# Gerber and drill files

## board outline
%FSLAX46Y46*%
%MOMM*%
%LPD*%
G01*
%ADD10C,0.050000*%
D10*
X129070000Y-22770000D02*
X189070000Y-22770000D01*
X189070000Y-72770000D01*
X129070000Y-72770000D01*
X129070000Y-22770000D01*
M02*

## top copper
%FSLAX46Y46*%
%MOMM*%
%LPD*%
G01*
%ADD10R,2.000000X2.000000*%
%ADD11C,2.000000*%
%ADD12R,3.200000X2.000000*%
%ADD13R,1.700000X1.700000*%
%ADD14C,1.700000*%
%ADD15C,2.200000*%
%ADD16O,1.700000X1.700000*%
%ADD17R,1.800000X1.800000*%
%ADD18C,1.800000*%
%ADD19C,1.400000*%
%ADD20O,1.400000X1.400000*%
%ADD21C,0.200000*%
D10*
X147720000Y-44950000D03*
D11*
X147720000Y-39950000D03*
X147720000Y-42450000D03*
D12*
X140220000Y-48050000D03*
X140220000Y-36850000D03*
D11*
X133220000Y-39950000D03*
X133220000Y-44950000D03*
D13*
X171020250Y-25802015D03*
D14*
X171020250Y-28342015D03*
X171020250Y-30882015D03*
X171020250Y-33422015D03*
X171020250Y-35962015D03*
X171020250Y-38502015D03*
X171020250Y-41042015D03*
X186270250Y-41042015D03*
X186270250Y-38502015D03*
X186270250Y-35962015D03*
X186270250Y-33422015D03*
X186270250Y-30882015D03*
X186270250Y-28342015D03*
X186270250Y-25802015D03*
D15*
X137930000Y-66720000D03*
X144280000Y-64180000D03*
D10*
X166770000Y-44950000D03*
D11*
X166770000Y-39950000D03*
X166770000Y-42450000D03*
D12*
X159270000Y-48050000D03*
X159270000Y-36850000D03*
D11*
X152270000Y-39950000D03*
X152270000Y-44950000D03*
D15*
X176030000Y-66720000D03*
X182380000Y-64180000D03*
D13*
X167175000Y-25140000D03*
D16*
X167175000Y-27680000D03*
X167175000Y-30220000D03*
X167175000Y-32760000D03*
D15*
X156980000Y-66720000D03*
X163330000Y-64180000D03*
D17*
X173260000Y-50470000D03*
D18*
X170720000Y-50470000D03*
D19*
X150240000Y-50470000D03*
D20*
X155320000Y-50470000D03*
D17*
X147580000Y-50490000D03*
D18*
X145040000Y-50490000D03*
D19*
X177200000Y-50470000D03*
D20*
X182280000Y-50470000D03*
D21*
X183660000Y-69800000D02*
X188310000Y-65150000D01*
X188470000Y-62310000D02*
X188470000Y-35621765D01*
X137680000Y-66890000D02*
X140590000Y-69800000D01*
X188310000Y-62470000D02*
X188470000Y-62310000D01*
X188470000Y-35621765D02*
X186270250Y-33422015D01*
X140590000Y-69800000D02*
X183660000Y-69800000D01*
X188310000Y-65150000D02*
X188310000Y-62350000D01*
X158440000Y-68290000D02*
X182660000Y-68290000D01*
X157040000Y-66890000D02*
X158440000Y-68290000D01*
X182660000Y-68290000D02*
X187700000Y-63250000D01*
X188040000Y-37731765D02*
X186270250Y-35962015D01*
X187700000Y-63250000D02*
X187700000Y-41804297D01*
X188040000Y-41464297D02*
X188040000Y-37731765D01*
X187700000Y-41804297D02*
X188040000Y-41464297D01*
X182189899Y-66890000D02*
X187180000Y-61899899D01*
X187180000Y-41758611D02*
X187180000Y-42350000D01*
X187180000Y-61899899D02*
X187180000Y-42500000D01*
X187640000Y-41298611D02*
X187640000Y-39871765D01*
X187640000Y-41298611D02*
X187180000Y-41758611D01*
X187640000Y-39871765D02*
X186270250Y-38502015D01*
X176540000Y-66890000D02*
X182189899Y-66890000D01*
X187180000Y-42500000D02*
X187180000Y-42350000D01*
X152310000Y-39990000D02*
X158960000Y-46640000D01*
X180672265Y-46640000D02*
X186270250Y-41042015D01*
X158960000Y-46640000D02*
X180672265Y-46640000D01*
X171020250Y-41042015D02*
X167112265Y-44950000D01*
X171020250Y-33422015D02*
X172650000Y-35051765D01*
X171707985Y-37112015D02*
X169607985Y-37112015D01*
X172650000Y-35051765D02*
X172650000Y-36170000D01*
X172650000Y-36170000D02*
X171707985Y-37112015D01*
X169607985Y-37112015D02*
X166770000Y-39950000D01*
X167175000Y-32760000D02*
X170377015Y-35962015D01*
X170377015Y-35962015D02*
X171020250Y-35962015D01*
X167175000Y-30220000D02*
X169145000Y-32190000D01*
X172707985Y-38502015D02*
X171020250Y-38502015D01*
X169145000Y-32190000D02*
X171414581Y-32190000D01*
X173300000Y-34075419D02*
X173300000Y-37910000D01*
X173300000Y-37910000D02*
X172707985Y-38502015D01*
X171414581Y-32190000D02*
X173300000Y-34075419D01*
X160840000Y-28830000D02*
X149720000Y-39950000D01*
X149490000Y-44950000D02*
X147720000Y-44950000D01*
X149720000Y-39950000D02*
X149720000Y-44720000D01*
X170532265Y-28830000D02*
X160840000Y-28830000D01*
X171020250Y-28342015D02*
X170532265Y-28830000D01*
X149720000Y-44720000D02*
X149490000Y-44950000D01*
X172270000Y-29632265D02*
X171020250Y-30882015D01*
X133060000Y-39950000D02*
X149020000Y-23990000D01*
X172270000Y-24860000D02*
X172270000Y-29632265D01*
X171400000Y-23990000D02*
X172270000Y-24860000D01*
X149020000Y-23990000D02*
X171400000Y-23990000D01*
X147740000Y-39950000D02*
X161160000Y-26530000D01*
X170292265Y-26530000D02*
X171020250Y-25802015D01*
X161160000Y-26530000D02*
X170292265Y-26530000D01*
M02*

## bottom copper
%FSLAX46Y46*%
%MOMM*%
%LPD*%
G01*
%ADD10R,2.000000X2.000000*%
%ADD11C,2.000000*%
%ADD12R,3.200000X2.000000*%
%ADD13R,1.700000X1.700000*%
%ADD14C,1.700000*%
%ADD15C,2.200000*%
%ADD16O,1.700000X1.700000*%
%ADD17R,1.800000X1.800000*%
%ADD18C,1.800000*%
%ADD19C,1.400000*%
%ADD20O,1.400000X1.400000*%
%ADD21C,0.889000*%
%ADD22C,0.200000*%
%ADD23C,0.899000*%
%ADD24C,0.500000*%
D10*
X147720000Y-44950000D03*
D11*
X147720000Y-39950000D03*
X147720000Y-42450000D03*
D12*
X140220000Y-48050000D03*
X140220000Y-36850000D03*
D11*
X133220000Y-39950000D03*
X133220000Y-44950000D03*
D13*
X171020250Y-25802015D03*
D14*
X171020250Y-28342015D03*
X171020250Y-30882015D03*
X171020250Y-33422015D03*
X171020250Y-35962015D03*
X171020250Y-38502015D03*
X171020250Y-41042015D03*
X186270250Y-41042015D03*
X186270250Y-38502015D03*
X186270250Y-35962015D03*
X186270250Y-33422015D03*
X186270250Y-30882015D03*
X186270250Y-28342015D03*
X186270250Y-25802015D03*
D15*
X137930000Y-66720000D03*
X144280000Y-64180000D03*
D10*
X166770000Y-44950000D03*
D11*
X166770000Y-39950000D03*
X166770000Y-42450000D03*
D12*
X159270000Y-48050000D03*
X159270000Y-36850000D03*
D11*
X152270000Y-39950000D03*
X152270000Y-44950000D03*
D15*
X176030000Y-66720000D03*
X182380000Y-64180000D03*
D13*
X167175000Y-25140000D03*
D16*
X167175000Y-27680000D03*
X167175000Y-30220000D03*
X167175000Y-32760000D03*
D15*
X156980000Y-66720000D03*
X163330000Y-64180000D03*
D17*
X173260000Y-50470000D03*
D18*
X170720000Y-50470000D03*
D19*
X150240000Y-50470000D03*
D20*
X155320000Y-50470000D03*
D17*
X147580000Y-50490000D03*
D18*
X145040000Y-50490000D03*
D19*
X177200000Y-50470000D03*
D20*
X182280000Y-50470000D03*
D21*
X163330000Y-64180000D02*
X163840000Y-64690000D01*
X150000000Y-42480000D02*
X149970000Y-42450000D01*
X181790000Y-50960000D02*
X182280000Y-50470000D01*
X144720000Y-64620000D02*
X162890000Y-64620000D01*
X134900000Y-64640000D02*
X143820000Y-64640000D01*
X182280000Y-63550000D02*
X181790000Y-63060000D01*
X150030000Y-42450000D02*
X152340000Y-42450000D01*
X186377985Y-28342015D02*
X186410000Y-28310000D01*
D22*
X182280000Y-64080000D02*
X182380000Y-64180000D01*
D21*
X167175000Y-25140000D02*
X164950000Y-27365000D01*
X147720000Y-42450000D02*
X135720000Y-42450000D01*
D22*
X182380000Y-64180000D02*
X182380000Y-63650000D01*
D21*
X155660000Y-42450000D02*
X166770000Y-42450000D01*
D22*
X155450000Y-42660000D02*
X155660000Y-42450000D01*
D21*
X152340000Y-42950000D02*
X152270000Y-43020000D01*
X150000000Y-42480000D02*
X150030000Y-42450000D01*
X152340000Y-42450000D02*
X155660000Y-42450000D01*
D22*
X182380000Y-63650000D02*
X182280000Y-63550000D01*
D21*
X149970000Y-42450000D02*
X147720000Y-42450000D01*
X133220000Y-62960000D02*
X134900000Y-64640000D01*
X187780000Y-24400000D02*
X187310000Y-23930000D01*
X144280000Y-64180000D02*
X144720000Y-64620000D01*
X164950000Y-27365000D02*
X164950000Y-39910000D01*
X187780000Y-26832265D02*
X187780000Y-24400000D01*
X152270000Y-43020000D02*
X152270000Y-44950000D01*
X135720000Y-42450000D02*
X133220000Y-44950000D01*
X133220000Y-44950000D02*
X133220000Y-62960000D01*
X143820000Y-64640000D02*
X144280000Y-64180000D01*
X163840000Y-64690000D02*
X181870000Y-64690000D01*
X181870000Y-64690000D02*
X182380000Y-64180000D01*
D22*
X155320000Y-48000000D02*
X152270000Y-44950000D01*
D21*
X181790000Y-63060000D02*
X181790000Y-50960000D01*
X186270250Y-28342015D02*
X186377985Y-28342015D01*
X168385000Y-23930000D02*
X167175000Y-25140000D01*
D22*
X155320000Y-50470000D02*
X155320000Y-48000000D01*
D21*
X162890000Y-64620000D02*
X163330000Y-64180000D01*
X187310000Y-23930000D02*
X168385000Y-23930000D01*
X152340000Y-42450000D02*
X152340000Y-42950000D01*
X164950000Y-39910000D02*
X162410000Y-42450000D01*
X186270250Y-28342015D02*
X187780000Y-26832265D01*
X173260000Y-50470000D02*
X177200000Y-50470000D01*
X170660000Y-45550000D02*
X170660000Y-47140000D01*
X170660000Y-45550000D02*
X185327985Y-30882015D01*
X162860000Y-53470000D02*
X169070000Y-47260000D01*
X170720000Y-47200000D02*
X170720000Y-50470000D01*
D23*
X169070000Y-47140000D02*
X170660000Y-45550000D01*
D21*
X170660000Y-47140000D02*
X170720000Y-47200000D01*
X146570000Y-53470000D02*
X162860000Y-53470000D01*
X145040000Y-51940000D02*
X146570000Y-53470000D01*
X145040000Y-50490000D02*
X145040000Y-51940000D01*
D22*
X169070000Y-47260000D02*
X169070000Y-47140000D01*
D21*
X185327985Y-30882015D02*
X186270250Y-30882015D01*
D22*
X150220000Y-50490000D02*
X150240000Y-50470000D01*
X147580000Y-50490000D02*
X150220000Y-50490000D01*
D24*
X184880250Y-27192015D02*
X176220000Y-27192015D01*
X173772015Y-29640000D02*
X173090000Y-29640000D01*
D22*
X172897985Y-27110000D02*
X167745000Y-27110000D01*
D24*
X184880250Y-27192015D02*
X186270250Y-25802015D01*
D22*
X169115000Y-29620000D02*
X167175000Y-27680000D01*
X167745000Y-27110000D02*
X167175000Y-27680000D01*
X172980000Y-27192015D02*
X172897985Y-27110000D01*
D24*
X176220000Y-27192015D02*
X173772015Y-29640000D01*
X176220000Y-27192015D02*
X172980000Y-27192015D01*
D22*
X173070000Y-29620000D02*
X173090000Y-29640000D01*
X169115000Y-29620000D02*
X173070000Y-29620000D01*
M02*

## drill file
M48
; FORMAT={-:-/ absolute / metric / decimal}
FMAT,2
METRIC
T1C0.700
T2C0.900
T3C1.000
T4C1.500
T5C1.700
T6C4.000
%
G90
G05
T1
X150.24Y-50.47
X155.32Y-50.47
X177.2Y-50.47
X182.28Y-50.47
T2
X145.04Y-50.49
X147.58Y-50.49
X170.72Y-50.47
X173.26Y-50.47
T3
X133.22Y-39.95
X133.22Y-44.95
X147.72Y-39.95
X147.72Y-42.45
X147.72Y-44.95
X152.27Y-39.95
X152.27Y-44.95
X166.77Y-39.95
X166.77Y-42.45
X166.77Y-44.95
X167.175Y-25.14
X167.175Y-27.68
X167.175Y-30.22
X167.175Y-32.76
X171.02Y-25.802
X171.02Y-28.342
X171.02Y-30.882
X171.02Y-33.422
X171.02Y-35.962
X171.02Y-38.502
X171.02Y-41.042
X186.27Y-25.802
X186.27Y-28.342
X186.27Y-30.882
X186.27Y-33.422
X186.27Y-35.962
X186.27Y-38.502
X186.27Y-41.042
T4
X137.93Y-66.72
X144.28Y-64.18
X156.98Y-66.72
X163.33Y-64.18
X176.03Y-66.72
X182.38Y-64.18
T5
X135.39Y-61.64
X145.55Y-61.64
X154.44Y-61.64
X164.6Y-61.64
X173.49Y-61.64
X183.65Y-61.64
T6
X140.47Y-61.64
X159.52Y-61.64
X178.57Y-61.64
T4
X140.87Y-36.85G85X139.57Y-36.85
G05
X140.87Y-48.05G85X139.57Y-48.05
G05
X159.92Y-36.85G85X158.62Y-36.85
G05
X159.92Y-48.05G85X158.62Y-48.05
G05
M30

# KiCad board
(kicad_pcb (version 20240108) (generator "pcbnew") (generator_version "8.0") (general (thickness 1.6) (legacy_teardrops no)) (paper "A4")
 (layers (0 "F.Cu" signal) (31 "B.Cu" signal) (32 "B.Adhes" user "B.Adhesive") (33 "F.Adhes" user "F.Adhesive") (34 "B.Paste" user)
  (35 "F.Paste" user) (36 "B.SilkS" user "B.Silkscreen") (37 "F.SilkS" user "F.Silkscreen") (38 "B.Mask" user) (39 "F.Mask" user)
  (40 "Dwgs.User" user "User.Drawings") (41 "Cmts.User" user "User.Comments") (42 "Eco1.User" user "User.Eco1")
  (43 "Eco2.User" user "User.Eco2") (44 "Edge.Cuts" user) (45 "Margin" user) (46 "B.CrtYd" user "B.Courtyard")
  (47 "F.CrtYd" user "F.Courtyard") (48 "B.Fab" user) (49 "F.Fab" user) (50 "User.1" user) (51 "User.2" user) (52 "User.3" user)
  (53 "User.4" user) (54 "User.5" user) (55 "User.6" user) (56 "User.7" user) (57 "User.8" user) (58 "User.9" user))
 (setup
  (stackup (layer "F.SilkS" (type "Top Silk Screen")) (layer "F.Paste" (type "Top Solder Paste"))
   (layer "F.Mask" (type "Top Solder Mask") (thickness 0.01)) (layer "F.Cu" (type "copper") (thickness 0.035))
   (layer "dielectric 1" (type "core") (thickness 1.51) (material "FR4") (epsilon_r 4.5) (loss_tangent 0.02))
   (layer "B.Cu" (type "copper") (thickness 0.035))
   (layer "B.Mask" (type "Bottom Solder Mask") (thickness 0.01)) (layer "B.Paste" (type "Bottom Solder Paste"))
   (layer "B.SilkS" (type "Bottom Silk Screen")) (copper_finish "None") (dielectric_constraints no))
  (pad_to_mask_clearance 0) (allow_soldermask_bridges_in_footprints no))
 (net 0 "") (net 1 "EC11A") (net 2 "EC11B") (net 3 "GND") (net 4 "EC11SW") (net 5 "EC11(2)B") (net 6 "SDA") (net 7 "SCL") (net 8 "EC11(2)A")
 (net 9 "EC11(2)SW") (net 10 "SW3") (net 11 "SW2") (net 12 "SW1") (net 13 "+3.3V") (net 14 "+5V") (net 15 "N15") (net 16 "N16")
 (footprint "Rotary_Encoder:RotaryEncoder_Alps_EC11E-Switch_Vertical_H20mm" (layer "F.Cu") (at 147.72 44.95 180)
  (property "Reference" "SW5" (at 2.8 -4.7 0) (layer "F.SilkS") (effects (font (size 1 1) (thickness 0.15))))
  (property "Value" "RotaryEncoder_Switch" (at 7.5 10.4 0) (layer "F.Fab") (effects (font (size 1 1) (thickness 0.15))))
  (pad "A" thru_hole rect (at 0 0 180) (size 2 2) (drill 1) (layers "*.Cu" "*.Mask") (remove_unused_layers no) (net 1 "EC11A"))
  (pad "B" thru_hole circle (at 0 5 180) (size 2 2) (drill 1) (layers "*.Cu" "*.Mask") (remove_unused_layers no) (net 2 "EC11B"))
  (pad "C" thru_hole circle (at 0 2.5 180) (size 2 2) (drill 1) (layers "*.Cu" "*.Mask") (remove_unused_layers no) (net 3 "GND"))
  (pad "MP" thru_hole rect (at 7.5 -3.1 180) (size 3.2 2) (drill oval 2.8 1.5) (layers "*.Cu" "*.Mask") (remove_unused_layers no))
  (pad "MP" thru_hole rect (at 7.5 8.1 180) (size 3.2 2) (drill oval 2.8 1.5) (layers "*.Cu" "*.Mask") (remove_unused_layers no))
  (pad "S1" thru_hole circle (at 14.5 5 180) (size 2 2) (drill 1) (layers "*.Cu" "*.Mask") (remove_unused_layers no) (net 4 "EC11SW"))
  (pad "S2" thru_hole circle (at 14.5 0 180) (size 2 2) (drill 1) (layers "*.Cu" "*.Mask") (remove_unused_layers no) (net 3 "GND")))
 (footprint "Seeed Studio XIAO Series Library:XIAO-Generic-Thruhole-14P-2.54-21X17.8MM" (layer "F.Cu") (at 178.64525 33.422015)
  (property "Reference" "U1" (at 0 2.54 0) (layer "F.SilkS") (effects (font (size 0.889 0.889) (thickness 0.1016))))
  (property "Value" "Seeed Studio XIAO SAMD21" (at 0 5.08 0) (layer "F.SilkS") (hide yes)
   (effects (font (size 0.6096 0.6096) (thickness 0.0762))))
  (pad "1" thru_hole rect (at -7.625 -7.62) (size 1.7 1.7) (drill 1) (layers "*.Cu" "*.Mask") (remove_unused_layers no) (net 2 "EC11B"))
  (pad "2" thru_hole circle (at -7.625 -5.08) (size 1.7 1.7) (drill 1) (layers "*.Cu" "*.Mask") (remove_unused_layers no) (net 1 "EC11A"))
  (pad "3" thru_hole circle (at -7.625 -2.54) (size 1.7 1.7) (drill 1) (layers "*.Cu" "*.Mask") (remove_unused_layers no) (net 4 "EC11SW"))
  (pad "4" thru_hole circle (at -7.625 0) (size 1.7 1.7) (drill 1) (layers "*.Cu" "*.Mask") (remove_unused_layers no) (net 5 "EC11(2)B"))
  (pad "5" thru_hole circle (at -7.625 2.54) (size 1.7 1.7) (drill 1) (layers "*.Cu" "*.Mask") (remove_unused_layers no) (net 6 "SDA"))
  (pad "6" thru_hole circle (at -7.625 5.08 180) (size 1.7 1.7) (drill 1) (layers "*.Cu" "*.Mask") (remove_unused_layers no) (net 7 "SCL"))
  (pad "7" thru_hole circle (at -7.625 7.62) (size 1.7 1.7) (drill 1) (layers "*.Cu" "*.Mask") (remove_unused_layers no) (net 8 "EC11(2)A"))
  (pad "8" thru_hole circle (at 7.625 7.62) (size 1.7 1.7) (drill 1) (layers "*.Cu" "*.Mask") (remove_unused_layers no) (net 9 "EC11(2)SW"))
  (pad "9" thru_hole circle (at 7.625 5.08) (size 1.7 1.7) (drill 1) (layers "*.Cu" "*.Mask") (remove_unused_layers no) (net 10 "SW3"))
  (pad "10" thru_hole circle (at 7.625 2.54) (size 1.7 1.7) (drill 1) (layers "*.Cu" "*.Mask") (remove_unused_layers no) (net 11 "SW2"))
  (pad "11" thru_hole circle (at 7.625 0) (size 1.7 1.7) (drill 1) (layers "*.Cu" "*.Mask") (remove_unused_layers no) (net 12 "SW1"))
  (pad "12" thru_hole circle (at 7.625 -2.54) (size 1.7 1.7) (drill 1) (layers "*.Cu" "*.Mask") (remove_unused_layers no) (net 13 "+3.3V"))
  (pad "13" thru_hole circle (at 7.625 -5.08) (size 1.7 1.7) (drill 1) (layers "*.Cu" "*.Mask") (remove_unused_layers no) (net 3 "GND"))
  (pad "14" thru_hole circle (at 7.625 -7.62) (size 1.7 1.7) (drill 1) (layers "*.Cu" "*.Mask") (remove_unused_layers no) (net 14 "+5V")))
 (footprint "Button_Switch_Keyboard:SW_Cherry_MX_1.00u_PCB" (layer "F.Cu") (at 137.93 66.72 180)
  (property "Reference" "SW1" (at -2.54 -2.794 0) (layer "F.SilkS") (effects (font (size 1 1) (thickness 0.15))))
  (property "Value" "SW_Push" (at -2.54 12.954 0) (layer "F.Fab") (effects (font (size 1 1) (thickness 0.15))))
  (pad "" np_thru_hole circle (at -7.62 5.08 180) (size 1.7 1.7) (drill 1.7) (layers "*.Cu" "*.Mask"))
  (pad "" np_thru_hole circle (at -2.54 5.08 180) (size 4 4) (drill 4) (layers "*.Cu" "*.Mask"))
  (pad "" np_thru_hole circle (at 2.54 5.08 180) (size 1.7 1.7) (drill 1.7) (layers "*.Cu" "*.Mask"))
  (pad "1" thru_hole circle (at 0 0 180) (size 2.2 2.2) (drill 1.5) (layers "*.Cu" "*.Mask") (remove_unused_layers no) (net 12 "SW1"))
  (pad "2" thru_hole circle (at -6.35 2.54 180) (size 2.2 2.2) (drill 1.5) (layers "*.Cu" "*.Mask") (remove_unused_layers no) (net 3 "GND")))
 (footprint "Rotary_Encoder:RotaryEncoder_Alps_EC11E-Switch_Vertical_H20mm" (layer "F.Cu") (at 166.77 44.95 180)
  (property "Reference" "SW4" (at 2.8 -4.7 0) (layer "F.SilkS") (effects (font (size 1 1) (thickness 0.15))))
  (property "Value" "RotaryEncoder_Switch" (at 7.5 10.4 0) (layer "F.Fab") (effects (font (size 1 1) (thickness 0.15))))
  (pad "A" thru_hole rect (at 0 0 180) (size 2 2) (drill 1) (layers "*.Cu" "*.Mask") (remove_unused_layers no) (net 8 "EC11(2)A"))
  (pad "B" thru_hole circle (at 0 5 180) (size 2 2) (drill 1) (layers "*.Cu" "*.Mask") (remove_unused_layers no) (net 5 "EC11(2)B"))
  (pad "C" thru_hole circle (at 0 2.5 180) (size 2 2) (drill 1) (layers "*.Cu" "*.Mask") (remove_unused_layers no) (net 3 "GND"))
  (pad "MP" thru_hole rect (at 7.5 -3.1 180) (size 3.2 2) (drill oval 2.8 1.5) (layers "*.Cu" "*.Mask") (remove_unused_layers no))
  (pad "MP" thru_hole rect (at 7.5 8.1 180) (size 3.2 2) (drill oval 2.8 1.5) (layers "*.Cu" "*.Mask") (remove_unused_layers no))
  (pad "S1" thru_hole circle (at 14.5 5 180) (size 2 2) (drill 1) (layers "*.Cu" "*.Mask") (remove_unused_layers no) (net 9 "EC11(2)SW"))
  (pad "S2" thru_hole circle (at 14.5 0 180) (size 2 2) (drill 1) (layers "*.Cu" "*.Mask") (remove_unused_layers no) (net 3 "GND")))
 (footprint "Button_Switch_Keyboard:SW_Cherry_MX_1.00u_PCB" (layer "F.Cu") (at 176.03 66.72 180)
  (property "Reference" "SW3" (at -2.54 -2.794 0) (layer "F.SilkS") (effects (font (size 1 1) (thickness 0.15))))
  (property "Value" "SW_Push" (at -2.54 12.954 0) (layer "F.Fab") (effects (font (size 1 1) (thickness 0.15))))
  (pad "" np_thru_hole circle (at -7.62 5.08 180) (size 1.7 1.7) (drill 1.7) (layers "*.Cu" "*.Mask"))
  (pad "" np_thru_hole circle (at -2.54 5.08 180) (size 4 4) (drill 4) (layers "*.Cu" "*.Mask"))
  (pad "" np_thru_hole circle (at 2.54 5.08 180) (size 1.7 1.7) (drill 1.7) (layers "*.Cu" "*.Mask"))
  (pad "1" thru_hole circle (at 0 0 180) (size 2.2 2.2) (drill 1.5) (layers "*.Cu" "*.Mask") (remove_unused_layers no) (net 10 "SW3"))
  (pad "2" thru_hole circle (at -6.35 2.54 180) (size 2.2 2.2) (drill 1.5) (layers "*.Cu" "*.Mask") (remove_unused_layers no) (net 3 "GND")))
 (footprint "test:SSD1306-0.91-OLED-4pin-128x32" (layer "F.Cu") (at 130.675 22.95)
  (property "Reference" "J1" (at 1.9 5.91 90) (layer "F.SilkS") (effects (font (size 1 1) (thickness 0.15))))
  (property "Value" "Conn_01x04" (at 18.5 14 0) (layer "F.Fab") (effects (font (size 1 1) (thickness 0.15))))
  (pad "1" thru_hole rect (at 36.5 2.19) (size 1.7 1.7) (drill 1) (layers "*.Cu" "*.Mask") (remove_unused_layers no) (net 3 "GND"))
  (pad "2" thru_hole oval (at 36.5 4.73) (size 1.7 1.7) (drill 1) (layers "*.Cu" "*.Mask") (remove_unused_layers no) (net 14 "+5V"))
  (pad "3" thru_hole oval (at 36.5 7.27) (size 1.7 1.7) (drill 1) (layers "*.Cu" "*.Mask") (remove_unused_layers no) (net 7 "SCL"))
  (pad "4" thru_hole oval (at 36.5 9.81) (size 1.7 1.7) (drill 1) (layers "*.Cu" "*.Mask") (remove_unused_layers no) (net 6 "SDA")))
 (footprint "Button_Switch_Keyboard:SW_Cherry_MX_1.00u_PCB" (layer "F.Cu") (at 156.98 66.72 180)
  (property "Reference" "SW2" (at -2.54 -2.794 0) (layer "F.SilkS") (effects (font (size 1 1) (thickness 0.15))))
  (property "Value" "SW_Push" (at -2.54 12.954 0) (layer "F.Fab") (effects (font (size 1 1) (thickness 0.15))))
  (pad "" np_thru_hole circle (at -7.62 5.08 180) (size 1.7 1.7) (drill 1.7) (layers "*.Cu" "*.Mask"))
  (pad "" np_thru_hole circle (at -2.54 5.08 180) (size 4 4) (drill 4) (layers "*.Cu" "*.Mask"))
  (pad "" np_thru_hole circle (at 2.54 5.08 180) (size 1.7 1.7) (drill 1.7) (layers "*.Cu" "*.Mask"))
  (pad "1" thru_hole circle (at 0 0 180) (size 2.2 2.2) (drill 1.5) (layers "*.Cu" "*.Mask") (remove_unused_layers no) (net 11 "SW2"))
  (pad "2" thru_hole circle (at -6.35 2.54 180) (size 2.2 2.2) (drill 1.5) (layers "*.Cu" "*.Mask") (remove_unused_layers no) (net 3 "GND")))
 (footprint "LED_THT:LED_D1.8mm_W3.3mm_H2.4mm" (layer "B.Cu") (at 173.26 50.47 180)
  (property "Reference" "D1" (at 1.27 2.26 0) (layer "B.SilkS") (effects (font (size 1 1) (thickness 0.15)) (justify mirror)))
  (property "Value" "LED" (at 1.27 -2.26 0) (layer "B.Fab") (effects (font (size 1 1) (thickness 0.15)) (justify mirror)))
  (pad "1" thru_hole rect (at 0 0 180) (size 1.8 1.8) (drill 0.9) (layers "*.Cu" "*.Mask") (remove_unused_layers no) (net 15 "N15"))
  (pad "2" thru_hole circle (at 2.54 0 180) (size 1.8 1.8) (drill 0.9) (layers "*.Cu" "*.Mask") (remove_unused_layers no) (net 13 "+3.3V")))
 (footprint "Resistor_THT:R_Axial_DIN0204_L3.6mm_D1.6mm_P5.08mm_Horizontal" (layer "B.Cu") (at 150.24 50.47)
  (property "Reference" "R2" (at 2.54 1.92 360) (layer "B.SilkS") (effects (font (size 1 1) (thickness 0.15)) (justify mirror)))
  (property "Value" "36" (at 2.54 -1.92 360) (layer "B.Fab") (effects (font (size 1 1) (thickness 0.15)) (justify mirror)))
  (pad "1" thru_hole circle (at 0 0) (size 1.4 1.4) (drill 0.7) (layers "*.Cu" "*.Mask") (remove_unused_layers no) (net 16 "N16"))
  (pad "2" thru_hole oval (at 5.08 0) (size 1.4 1.4) (drill 0.7) (layers "*.Cu" "*.Mask") (remove_unused_layers no) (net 3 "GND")))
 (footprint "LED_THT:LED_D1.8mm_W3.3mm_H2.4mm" (layer "B.Cu") (at 147.58 50.49 180)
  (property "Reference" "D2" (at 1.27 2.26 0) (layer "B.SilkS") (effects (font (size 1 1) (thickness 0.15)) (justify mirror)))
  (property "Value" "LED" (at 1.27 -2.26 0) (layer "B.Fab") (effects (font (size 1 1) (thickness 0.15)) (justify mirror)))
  (pad "1" thru_hole rect (at 0 0 180) (size 1.8 1.8) (drill 0.9) (layers "*.Cu" "*.Mask") (remove_unused_layers no) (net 16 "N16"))
  (pad "2" thru_hole circle (at 2.54 0 180) (size 1.8 1.8) (drill 0.9) (layers "*.Cu" "*.Mask") (remove_unused_layers no) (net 13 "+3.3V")))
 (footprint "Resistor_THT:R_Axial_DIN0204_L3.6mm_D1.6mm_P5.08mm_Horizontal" (layer "B.Cu") (at 177.2 50.47)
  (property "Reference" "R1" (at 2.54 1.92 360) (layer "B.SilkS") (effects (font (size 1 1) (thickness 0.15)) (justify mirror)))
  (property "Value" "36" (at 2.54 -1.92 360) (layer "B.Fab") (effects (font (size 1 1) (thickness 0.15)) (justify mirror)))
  (pad "1" thru_hole circle (at 0 0) (size 1.4 1.4) (drill 0.7) (layers "*.Cu" "*.Mask") (remove_unused_layers no) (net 15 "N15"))
  (pad "2" thru_hole oval (at 5.08 0) (size 1.4 1.4) (drill 0.7) (layers "*.Cu" "*.Mask") (remove_unused_layers no) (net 3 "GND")))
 (gr_rect (start 129.07 22.77) (end 189.07 72.77) (stroke (width 0.05) (type default)) (fill none) (layer "Edge.Cuts"))
 (segment (start 163.33 64.18) (end 163.84 64.69) (width 0.889) (layer "B.Cu") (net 3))
 (segment (start 150 42.48) (end 149.97 42.45) (width 0.889) (layer "B.Cu") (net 3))
 (segment (start 181.79 50.96) (end 182.28 50.47) (width 0.889) (layer "B.Cu") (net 3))
 (segment (start 144.72 64.62) (end 162.89 64.62) (width 0.889) (layer "B.Cu") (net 3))
 (segment (start 134.9 64.64) (end 143.82 64.64) (width 0.889) (layer "B.Cu") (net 3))
 (segment (start 182.28 63.55) (end 181.79 63.06) (width 0.889) (layer "B.Cu") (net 3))
 (segment (start 150.03 42.45) (end 152.34 42.45) (width 0.889) (layer "B.Cu") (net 3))
 (segment (start 186.377985 28.342015) (end 186.41 28.31) (width 0.889) (layer "B.Cu") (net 3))
 (segment (start 182.28 64.08) (end 182.38 64.18) (width 0.2) (layer "B.Cu") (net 3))
 (segment (start 167.175 25.14) (end 164.95 27.365) (width 0.889) (layer "B.Cu") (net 3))
 (segment (start 147.72 42.45) (end 135.72 42.45) (width 0.889) (layer "B.Cu") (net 3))
 (segment (start 182.38 64.18) (end 182.38 63.65) (width 0.2) (layer "B.Cu") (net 3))
 (segment (start 155.66 42.45) (end 166.77 42.45) (width 0.889) (layer "B.Cu") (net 3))
 (segment (start 155.45 42.66) (end 155.66 42.45) (width 0.2) (layer "B.Cu") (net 3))
 (segment (start 152.34 42.95) (end 152.27 43.02) (width 0.889) (layer "B.Cu") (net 3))
 (segment (start 150 42.48) (end 150.03 42.45) (width 0.889) (layer "B.Cu") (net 3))
 (segment (start 152.34 42.45) (end 155.66 42.45) (width 0.889) (layer "B.Cu") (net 3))
 (segment (start 182.38 63.65) (end 182.28 63.55) (width 0.2) (layer "B.Cu") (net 3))
 (segment (start 149.97 42.45) (end 147.72 42.45) (width 0.889) (layer "B.Cu") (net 3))
 (segment (start 133.22 62.96) (end 134.9 64.64) (width 0.889) (layer "B.Cu") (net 3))
 (segment (start 187.78 24.4) (end 187.31 23.93) (width 0.889) (layer "B.Cu") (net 3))
 (segment (start 144.28 64.18) (end 144.72 64.62) (width 0.889) (layer "B.Cu") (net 3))
 (segment (start 164.95 27.365) (end 164.95 39.91) (width 0.889) (layer "B.Cu") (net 3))
 (segment (start 187.78 26.832265) (end 187.78 24.4) (width 0.889) (layer "B.Cu") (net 3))
 (segment (start 152.27 43.02) (end 152.27 44.95) (width 0.889) (layer "B.Cu") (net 3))
 (segment (start 135.72 42.45) (end 133.22 44.95) (width 0.889) (layer "B.Cu") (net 3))
 (segment (start 133.22 44.95) (end 133.22 62.96) (width 0.889) (layer "B.Cu") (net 3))
 (segment (start 143.82 64.64) (end 144.28 64.18) (width 0.889) (layer "B.Cu") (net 3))
 (segment (start 163.84 64.69) (end 181.87 64.69) (width 0.889) (layer "B.Cu") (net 3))
 (segment (start 181.87 64.69) (end 182.38 64.18) (width 0.889) (layer "B.Cu") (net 3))
 (segment (start 155.32 48) (end 152.27 44.95) (width 0.2) (layer "B.Cu") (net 3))
 (segment (start 181.79 63.06) (end 181.79 50.96) (width 0.889) (layer "B.Cu") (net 3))
 (segment (start 186.27025 28.342015) (end 186.377985 28.342015) (width 0.889) (layer "B.Cu") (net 3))
 (segment (start 168.385 23.93) (end 167.175 25.14) (width 0.889) (layer "B.Cu") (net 3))
 (segment (start 155.32 50.47) (end 155.32 48) (width 0.2) (layer "B.Cu") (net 3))
 (segment (start 162.89 64.62) (end 163.33 64.18) (width 0.889) (layer "B.Cu") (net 3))
 (segment (start 187.31 23.93) (end 168.385 23.93) (width 0.889) (layer "B.Cu") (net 3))
 (segment (start 152.34 42.45) (end 152.34 42.95) (width 0.889) (layer "B.Cu") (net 3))
 (segment (start 164.95 39.91) (end 162.41 42.45) (width 0.889) (layer "B.Cu") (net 3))
 (segment (start 186.27025 28.342015) (end 187.78 26.832265) (width 0.889) (layer "B.Cu") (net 3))
 (segment (start 173.26 50.47) (end 177.2 50.47) (width 0.889) (layer "B.Cu") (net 15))
 (segment (start 170.66 45.55) (end 170.66 47.14) (width 0.889) (layer "B.Cu") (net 13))
 (segment (start 170.66 45.55) (end 185.327985 30.882015) (width 0.889) (layer "B.Cu") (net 13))
 (segment (start 162.86 53.47) (end 169.07 47.26) (width 0.889) (layer "B.Cu") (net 13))
 (segment (start 170.72 47.2) (end 170.72 50.47) (width 0.889) (layer "B.Cu") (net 13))
 (segment (start 169.07 47.14) (end 170.66 45.55) (width 0.899) (layer "B.Cu") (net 13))
 (segment (start 170.66 47.14) (end 170.72 47.2) (width 0.889) (layer "B.Cu") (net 13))
 (segment (start 146.57 53.47) (end 162.86 53.47) (width 0.889) (layer "B.Cu") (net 13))
 (segment (start 145.04 51.94) (end 146.57 53.47) (width 0.889) (layer "B.Cu") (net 13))
 (segment (start 145.04 50.49) (end 145.04 51.94) (width 0.889) (layer "B.Cu") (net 13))
 (segment (start 169.07 47.26) (end 169.07 47.14) (width 0.2) (layer "B.Cu") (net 13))
 (segment (start 185.327985 30.882015) (end 186.27025 30.882015) (width 0.889) (layer "B.Cu") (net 13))
 (segment (start 150.22 50.49) (end 150.24 50.47) (width 0.2) (layer "B.Cu") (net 16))
 (segment (start 147.58 50.49) (end 150.22 50.49) (width 0.2) (layer "B.Cu") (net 16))
 (segment (start 183.66 69.8) (end 188.31 65.15) (width 0.2) (layer "F.Cu") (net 12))
 (segment (start 188.47 62.31) (end 188.47 35.621765) (width 0.2) (layer "F.Cu") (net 12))
 (segment (start 137.68 66.89) (end 140.59 69.8) (width 0.2) (layer "F.Cu") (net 12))
 (segment (start 188.31 62.47) (end 188.47 62.31) (width 0.2) (layer "F.Cu") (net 12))
 (segment (start 188.47 35.621765) (end 186.27025 33.422015) (width 0.2) (layer "F.Cu") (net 12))
 (segment (start 140.59 69.8) (end 183.66 69.8) (width 0.2) (layer "F.Cu") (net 12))
 (segment (start 188.31 65.15) (end 188.31 62.35) (width 0.2) (layer "F.Cu") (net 12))
 (segment (start 158.44 68.29) (end 182.66 68.29) (width 0.2) (layer "F.Cu") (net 11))
 (segment (start 157.04 66.89) (end 158.44 68.29) (width 0.2) (layer "F.Cu") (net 11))
 (segment (start 182.66 68.29) (end 187.7 63.25) (width 0.2) (layer "F.Cu") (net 11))
 (segment (start 188.04 37.731765) (end 186.27025 35.962015) (width 0.2) (layer "F.Cu") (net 11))
 (segment (start 187.7 63.25) (end 187.7 41.804297) (width 0.2) (layer "F.Cu") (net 11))
 (segment (start 188.04 41.464297) (end 188.04 37.731765) (width 0.2) (layer "F.Cu") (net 11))
 (segment (start 187.7 41.804297) (end 188.04 41.464297) (width 0.2) (layer "F.Cu") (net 11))
 (segment (start 182.189899 66.89) (end 187.18 61.899899) (width 0.2) (layer "F.Cu") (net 10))
 (segment (start 187.18 41.758611) (end 187.18 42.35) (width 0.2) (layer "F.Cu") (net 10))
 (segment (start 187.18 61.899899) (end 187.18 42.5) (width 0.2) (layer "F.Cu") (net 10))
 (segment (start 187.64 41.298611) (end 187.64 39.871765) (width 0.2) (layer "F.Cu") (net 10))
 (segment (start 187.64 41.298611) (end 187.18 41.758611) (width 0.2) (layer "F.Cu") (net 10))
 (segment (start 187.64 39.871765) (end 186.27025 38.502015) (width 0.2) (layer "F.Cu") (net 10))
 (segment (start 176.54 66.89) (end 182.189899 66.89) (width 0.2) (layer "F.Cu") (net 10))
 (segment (start 187.18 42.5) (end 187.18 42.35) (width 0.2) (layer "F.Cu") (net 10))
 (segment (start 152.31 39.99) (end 158.96 46.64) (width 0.2) (layer "F.Cu") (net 9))
 (segment (start 180.672265 46.64) (end 186.27025 41.042015) (width 0.2) (layer "F.Cu") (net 9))
 (segment (start 158.96 46.64) (end 180.672265 46.64) (width 0.2) (layer "F.Cu") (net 9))
 (segment (start 171.02025 41.042015) (end 167.112265 44.95) (width 0.2) (layer "F.Cu") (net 8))
 (segment (start 171.02025 33.422015) (end 172.65 35.051765) (width 0.2) (layer "F.Cu") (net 5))
 (segment (start 171.707985 37.112015) (end 169.607985 37.112015) (width 0.2) (layer "F.Cu") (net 5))
 (segment (start 172.65 35.051765) (end 172.65 36.17) (width 0.2) (layer "F.Cu") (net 5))
 (segment (start 172.65 36.17) (end 171.707985 37.112015) (width 0.2) (layer "F.Cu") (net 5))
 (segment (start 169.607985 37.112015) (end 166.77 39.95) (width 0.2) (layer "F.Cu") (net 5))
 (segment (start 184.88025 27.192015) (end 176.22 27.192015) (width 0.5) (layer "B.Cu") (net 14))
 (segment (start 173.772015 29.64) (end 173.09 29.64) (width 0.5) (layer "B.Cu") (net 14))
 (segment (start 172.897985 27.11) (end 167.745 27.11) (width 0.2) (layer "B.Cu") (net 14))
 (segment (start 184.88025 27.192015) (end 186.27025 25.802015) (width 0.5) (layer "B.Cu") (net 14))
 (segment (start 169.115 29.62) (end 167.175 27.68) (width 0.2) (layer "B.Cu") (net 14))
 (segment (start 167.745 27.11) (end 167.175 27.68) (width 0.2) (layer "B.Cu") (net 14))
 (segment (start 172.98 27.192015) (end 172.897985 27.11) (width 0.2) (layer "B.Cu") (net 14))
 (segment (start 176.22 27.192015) (end 173.772015 29.64) (width 0.5) (layer "B.Cu") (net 14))
 (segment (start 176.22 27.192015) (end 172.98 27.192015) (width 0.5) (layer "B.Cu") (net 14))
 (segment (start 173.07 29.62) (end 173.09 29.64) (width 0.2) (layer "B.Cu") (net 14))
 (segment (start 169.115 29.62) (end 173.07 29.62) (width 0.2) (layer "B.Cu") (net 14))
 (segment (start 167.175 32.76) (end 170.377015 35.962015) (width 0.2) (layer "F.Cu") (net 6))
 (segment (start 170.377015 35.962015) (end 171.02025 35.962015) (width 0.2) (layer "F.Cu") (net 6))
 (segment (start 167.175 30.22) (end 169.145 32.19) (width 0.2) (layer "F.Cu") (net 7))
 (segment (start 172.707985 38.502015) (end 171.02025 38.502015) (width 0.2) (layer "F.Cu") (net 7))
 (segment (start 169.145 32.19) (end 171.414581 32.19) (width 0.2) (layer "F.Cu") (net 7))
 (segment (start 173.3 34.075419) (end 173.3 37.91) (width 0.2) (layer "F.Cu") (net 7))
 (segment (start 173.3 37.91) (end 172.707985 38.502015) (width 0.2) (layer "F.Cu") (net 7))
 (segment (start 171.414581 32.19) (end 173.3 34.075419) (width 0.2) (layer "F.Cu") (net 7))
 (segment (start 160.84 28.83) (end 149.72 39.95) (width 0.2) (layer "F.Cu") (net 1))
 (segment (start 149.49 44.95) (end 147.72 44.95) (width 0.2) (layer "F.Cu") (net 1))
 (segment (start 149.72 39.95) (end 149.72 44.72) (width 0.2) (layer "F.Cu") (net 1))
 (segment (start 170.532265 28.83) (end 160.84 28.83) (width 0.2) (layer "F.Cu") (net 1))
 (segment (start 171.02025 28.342015) (end 170.532265 28.83) (width 0.2) (layer "F.Cu") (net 1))
 (segment (start 149.72 44.72) (end 149.49 44.95) (width 0.2) (layer "F.Cu") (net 1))
 (segment (start 172.27 29.632265) (end 171.02025 30.882015) (width 0.2) (layer "F.Cu") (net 4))
 (segment (start 133.06 39.95) (end 149.02 23.99) (width 0.2) (layer "F.Cu") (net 4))
 (segment (start 172.27 24.86) (end 172.27 29.632265) (width 0.2) (layer "F.Cu") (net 4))
 (segment (start 171.4 23.99) (end 172.27 24.86) (width 0.2) (layer "F.Cu") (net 4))
 (segment (start 149.02 23.99) (end 171.4 23.99) (width 0.2) (layer "F.Cu") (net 4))
 (segment (start 147.74 39.95) (end 161.16 26.53) (width 0.2) (layer "F.Cu") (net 2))
 (segment (start 170.292265 26.53) (end 171.02025 25.802015) (width 0.2) (layer "F.Cu") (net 2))
 (segment (start 161.16 26.53) (end 170.292265 26.53) (width 0.2) (layer "F.Cu") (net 2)))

